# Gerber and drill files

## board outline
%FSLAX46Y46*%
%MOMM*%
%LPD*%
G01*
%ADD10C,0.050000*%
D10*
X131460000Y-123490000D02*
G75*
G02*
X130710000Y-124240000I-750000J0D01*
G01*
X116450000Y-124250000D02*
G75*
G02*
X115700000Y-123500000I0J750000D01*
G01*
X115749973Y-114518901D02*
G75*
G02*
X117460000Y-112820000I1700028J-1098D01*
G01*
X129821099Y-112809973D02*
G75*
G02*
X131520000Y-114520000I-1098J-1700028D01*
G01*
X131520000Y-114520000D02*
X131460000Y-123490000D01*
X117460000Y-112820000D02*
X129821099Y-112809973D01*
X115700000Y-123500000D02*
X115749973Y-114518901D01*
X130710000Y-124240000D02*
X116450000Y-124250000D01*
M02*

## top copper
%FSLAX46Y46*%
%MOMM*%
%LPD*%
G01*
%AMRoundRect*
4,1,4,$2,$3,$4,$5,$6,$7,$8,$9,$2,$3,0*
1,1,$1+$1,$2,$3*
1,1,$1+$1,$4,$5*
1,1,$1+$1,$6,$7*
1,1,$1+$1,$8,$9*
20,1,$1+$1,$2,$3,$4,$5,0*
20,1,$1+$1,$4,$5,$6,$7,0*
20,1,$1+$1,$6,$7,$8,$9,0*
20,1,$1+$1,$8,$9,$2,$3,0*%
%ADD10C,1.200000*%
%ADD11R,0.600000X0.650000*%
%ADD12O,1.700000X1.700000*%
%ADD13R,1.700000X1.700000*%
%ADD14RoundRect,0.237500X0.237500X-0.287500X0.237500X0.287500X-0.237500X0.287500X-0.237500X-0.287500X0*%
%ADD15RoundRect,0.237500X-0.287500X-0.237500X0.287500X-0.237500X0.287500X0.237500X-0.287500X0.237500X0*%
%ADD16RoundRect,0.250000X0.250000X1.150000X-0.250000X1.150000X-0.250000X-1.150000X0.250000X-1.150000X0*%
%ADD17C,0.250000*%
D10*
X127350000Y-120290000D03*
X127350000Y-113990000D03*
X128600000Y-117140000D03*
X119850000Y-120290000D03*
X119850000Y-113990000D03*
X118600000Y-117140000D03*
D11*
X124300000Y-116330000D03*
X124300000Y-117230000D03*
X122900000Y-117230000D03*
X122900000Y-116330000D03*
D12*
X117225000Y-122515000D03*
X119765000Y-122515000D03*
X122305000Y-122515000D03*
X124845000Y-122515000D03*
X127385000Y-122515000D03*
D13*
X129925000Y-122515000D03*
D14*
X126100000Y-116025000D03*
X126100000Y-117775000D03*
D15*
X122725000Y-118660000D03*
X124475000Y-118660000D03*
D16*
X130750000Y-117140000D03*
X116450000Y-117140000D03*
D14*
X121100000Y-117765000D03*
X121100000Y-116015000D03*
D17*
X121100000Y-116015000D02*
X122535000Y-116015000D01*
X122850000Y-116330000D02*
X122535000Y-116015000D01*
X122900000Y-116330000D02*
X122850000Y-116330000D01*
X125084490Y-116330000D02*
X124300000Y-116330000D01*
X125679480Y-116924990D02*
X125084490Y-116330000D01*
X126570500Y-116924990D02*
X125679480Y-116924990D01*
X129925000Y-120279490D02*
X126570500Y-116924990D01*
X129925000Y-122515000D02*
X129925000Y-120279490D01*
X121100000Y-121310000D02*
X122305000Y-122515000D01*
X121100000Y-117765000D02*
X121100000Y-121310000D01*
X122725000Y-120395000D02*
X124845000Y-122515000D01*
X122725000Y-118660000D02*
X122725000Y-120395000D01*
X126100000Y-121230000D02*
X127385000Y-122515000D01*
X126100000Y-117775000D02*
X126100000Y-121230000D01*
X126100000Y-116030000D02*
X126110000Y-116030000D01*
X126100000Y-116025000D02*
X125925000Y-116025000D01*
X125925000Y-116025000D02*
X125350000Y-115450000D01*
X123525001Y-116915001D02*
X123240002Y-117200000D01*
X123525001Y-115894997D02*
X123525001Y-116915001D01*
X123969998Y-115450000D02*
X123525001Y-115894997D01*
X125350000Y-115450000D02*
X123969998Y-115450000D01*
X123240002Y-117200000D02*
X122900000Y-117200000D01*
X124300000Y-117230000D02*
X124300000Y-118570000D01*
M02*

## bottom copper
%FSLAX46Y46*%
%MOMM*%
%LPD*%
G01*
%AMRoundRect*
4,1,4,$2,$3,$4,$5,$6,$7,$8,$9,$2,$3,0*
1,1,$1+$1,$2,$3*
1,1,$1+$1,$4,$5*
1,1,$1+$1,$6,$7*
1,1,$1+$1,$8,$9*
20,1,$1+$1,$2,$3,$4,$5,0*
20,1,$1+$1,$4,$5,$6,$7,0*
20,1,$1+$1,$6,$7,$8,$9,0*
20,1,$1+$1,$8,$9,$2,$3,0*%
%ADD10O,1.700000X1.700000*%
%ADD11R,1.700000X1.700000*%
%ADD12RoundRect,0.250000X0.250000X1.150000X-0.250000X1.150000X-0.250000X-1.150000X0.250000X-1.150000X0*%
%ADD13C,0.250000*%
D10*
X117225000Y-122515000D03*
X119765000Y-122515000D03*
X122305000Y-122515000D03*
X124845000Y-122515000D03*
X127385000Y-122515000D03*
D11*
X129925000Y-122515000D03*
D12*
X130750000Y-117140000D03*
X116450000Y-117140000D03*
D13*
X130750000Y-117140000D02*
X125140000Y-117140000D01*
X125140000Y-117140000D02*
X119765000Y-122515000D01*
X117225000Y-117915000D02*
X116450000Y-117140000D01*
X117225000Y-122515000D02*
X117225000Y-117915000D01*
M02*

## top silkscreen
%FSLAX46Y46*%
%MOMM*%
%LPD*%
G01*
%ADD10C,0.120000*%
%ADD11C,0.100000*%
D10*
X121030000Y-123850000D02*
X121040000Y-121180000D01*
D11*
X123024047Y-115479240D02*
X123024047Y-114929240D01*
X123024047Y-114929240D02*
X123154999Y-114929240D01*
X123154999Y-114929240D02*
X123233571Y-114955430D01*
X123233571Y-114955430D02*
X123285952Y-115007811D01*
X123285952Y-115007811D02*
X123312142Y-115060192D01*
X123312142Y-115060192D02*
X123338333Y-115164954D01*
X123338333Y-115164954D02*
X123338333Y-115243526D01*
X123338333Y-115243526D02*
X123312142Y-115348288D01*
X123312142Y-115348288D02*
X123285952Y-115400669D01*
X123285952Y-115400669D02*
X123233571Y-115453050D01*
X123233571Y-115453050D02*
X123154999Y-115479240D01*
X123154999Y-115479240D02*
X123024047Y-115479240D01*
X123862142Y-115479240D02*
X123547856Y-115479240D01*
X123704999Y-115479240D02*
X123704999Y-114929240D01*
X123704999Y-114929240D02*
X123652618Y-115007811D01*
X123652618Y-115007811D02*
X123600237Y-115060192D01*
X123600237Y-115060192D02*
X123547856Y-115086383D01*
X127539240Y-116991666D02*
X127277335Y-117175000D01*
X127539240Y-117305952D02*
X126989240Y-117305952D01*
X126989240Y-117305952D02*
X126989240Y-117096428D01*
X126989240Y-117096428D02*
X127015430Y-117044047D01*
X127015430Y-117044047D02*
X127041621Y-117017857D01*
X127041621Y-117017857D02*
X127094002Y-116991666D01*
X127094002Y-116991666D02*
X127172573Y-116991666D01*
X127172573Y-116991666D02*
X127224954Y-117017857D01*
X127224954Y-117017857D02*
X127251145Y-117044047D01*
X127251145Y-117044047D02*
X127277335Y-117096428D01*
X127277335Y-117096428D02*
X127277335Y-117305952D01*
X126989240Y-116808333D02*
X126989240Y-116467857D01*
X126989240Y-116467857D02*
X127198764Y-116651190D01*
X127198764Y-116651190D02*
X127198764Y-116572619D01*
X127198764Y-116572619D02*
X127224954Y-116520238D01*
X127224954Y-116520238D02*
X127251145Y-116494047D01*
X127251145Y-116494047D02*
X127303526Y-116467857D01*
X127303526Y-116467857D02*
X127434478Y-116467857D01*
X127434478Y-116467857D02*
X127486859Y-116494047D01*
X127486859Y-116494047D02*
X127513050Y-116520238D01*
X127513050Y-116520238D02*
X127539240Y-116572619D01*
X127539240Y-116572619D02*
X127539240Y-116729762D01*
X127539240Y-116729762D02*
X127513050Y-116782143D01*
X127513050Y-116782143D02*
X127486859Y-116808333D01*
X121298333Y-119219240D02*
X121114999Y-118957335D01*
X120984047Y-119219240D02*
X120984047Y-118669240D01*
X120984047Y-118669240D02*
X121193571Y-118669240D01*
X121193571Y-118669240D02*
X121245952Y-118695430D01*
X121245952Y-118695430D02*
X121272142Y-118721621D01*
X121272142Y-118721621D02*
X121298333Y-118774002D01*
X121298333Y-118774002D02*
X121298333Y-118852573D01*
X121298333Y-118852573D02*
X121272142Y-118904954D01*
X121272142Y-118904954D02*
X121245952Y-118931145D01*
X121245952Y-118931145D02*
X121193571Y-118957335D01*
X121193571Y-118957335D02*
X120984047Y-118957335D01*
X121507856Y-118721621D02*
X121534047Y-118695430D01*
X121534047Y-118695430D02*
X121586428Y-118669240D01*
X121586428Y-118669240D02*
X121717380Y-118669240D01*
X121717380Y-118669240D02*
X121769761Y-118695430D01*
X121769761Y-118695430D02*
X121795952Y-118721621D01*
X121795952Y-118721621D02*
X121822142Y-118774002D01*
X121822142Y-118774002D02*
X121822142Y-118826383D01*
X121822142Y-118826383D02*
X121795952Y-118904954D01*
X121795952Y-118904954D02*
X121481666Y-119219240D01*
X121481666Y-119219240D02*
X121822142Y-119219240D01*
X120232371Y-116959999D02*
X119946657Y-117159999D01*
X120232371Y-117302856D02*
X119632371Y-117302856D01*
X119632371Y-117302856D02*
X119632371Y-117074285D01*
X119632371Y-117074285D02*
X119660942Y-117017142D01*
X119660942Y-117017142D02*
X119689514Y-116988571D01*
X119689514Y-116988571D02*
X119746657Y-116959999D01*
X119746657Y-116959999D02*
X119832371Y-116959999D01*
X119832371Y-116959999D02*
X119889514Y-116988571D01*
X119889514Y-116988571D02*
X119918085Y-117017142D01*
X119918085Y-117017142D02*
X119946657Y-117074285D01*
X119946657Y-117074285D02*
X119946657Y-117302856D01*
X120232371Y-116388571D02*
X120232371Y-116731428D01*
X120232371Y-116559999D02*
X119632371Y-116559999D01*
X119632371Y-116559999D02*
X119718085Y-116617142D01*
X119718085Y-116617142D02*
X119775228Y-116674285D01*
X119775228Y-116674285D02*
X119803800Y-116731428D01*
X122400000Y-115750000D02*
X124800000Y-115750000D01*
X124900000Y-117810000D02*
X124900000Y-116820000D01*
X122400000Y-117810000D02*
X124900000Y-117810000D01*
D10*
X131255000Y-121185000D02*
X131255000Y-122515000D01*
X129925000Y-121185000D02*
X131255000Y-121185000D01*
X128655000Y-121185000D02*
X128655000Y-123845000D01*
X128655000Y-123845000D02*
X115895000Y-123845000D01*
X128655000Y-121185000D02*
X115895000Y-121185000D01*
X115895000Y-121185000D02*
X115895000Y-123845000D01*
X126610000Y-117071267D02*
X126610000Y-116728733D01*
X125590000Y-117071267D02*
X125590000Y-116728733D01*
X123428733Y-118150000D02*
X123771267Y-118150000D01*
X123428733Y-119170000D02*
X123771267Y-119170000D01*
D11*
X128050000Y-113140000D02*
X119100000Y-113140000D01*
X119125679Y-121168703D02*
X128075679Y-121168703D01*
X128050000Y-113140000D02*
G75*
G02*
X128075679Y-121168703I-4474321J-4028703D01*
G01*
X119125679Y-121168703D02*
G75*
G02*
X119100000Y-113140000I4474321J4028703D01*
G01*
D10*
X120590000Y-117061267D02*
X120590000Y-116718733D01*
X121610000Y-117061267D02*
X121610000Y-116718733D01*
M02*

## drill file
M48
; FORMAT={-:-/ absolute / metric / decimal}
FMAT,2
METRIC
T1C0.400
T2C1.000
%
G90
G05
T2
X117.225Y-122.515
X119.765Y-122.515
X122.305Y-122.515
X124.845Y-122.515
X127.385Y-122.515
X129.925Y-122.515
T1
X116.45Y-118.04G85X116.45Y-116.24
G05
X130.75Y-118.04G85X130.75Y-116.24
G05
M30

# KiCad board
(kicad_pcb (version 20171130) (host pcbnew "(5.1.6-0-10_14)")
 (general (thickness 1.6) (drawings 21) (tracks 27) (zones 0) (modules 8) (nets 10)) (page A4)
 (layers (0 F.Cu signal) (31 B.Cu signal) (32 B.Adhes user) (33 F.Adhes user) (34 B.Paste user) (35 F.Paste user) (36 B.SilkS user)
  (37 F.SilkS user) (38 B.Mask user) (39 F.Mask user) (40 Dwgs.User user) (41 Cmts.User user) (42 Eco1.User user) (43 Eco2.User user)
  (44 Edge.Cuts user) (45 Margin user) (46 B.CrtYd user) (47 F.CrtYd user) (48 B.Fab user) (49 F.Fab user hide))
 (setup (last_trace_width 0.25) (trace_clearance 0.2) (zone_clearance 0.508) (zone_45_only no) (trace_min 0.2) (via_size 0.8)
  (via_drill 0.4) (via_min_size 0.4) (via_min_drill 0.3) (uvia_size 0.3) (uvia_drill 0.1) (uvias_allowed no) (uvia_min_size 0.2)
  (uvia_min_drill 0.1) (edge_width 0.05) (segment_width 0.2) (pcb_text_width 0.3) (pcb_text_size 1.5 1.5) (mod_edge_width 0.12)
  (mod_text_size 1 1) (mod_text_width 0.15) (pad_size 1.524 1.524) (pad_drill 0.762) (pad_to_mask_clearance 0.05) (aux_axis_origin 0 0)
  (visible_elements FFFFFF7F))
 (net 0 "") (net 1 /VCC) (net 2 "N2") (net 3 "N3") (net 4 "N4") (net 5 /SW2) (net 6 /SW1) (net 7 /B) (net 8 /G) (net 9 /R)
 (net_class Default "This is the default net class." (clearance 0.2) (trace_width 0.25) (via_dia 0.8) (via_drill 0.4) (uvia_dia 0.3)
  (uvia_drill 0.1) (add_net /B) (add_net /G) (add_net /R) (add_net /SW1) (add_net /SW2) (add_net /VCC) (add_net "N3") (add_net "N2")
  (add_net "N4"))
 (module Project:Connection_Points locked (layer F.Cu) (at 123.6 117.14)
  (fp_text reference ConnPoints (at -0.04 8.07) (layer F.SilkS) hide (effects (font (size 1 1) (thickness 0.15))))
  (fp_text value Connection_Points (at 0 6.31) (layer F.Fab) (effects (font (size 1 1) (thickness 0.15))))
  (pad "" smd circle (at 3.75 3.15) (size 1.2 1.2) (layers F.Cu F.Paste F.Mask))
  (pad "" smd circle (at 3.75 -3.15) (size 1.2 1.2) (layers F.Cu F.Paste F.Mask))
  (pad "" smd circle (at 5 0) (size 1.2 1.2) (layers F.Cu F.Paste F.Mask))
  (pad "" smd circle (at -3.75 3.15) (size 1.2 1.2) (layers F.Cu F.Paste F.Mask))
  (pad "" smd circle (at -3.75 -3.15) (size 1.2 1.2) (layers F.Cu F.Paste F.Mask))
  (pad "" smd circle (at -5 0) (size 1.2 1.2) (layers F.Cu F.Paste F.Mask)))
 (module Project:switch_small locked (layer B.Cu) (at 118.42 120.41 180)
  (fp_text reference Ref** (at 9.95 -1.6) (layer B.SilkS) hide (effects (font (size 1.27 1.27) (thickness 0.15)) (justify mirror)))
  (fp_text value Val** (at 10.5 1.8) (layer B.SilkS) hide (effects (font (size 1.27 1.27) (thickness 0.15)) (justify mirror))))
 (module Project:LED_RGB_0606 (layer F.Cu) (at 123.6 116.78)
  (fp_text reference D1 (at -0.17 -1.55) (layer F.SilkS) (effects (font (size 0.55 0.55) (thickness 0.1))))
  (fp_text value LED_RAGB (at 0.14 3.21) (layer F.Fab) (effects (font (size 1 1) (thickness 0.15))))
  (fp_line (start -1.2 -1.03) (end 1.2 -1.03) (layer F.SilkS) (width 0.1))
  (fp_line (start 1.3 1.03) (end 1.3 0.04) (layer F.SilkS) (width 0.1))
  (fp_line (start -1.2 1.03) (end 1.3 1.03) (layer F.SilkS) (width 0.1))
  (pad 4 smd rect (at 0.7 -0.45) (size 0.6 0.65) (layers F.Cu F.Paste F.Mask) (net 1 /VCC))
  (pad 2 smd rect (at 0.7 0.45) (size 0.6 0.65) (layers F.Cu F.Paste F.Mask) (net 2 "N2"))
  (pad 1 smd rect (at -0.7 0.45) (size 0.6 0.65) (layers F.Cu F.Paste F.Mask) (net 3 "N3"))
  (pad 3 smd rect (at -0.7 -0.45) (size 0.6 0.65) (layers F.Cu F.Paste F.Mask) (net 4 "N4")))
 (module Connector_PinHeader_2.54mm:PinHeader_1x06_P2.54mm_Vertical (layer F.Cu) (at 129.925 122.515 270)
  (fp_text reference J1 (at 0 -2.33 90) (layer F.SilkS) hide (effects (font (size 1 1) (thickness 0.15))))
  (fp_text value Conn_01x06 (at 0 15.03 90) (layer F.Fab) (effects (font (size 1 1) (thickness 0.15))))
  (fp_line (start -1.33 -1.33) (end 0 -1.33) (layer F.SilkS) (width 0.12))
  (fp_line (start -1.33 0) (end -1.33 -1.33) (layer F.SilkS) (width 0.12))
  (fp_line (start -1.33 1.27) (end 1.33 1.27) (layer F.SilkS) (width 0.12))
  (fp_line (start 1.33 1.27) (end 1.33 14.03) (layer F.SilkS) (width 0.12))
  (fp_line (start -1.33 1.27) (end -1.33 14.03) (layer F.SilkS) (width 0.12))
  (fp_line (start -1.33 14.03) (end 1.33 14.03) (layer F.SilkS) (width 0.12))
  (pad 6 thru_hole oval (at 0 12.7 270) (size 1.7 1.7) (drill 1) (layers *.Cu *.Mask) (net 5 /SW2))
  (pad 5 thru_hole oval (at 0 10.16 270) (size 1.7 1.7) (drill 1) (layers *.Cu *.Mask) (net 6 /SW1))
  (pad 4 thru_hole oval (at 0 7.62 270) (size 1.7 1.7) (drill 1) (layers *.Cu *.Mask) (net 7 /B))
  (pad 3 thru_hole oval (at 0 5.08 270) (size 1.7 1.7) (drill 1) (layers *.Cu *.Mask) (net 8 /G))
  (pad 2 thru_hole oval (at 0 2.54 270) (size 1.7 1.7) (drill 1) (layers *.Cu *.Mask) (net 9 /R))
  (pad 1 thru_hole rect (at 0 0 270) (size 1.7 1.7) (drill 1) (layers *.Cu *.Mask) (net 1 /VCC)))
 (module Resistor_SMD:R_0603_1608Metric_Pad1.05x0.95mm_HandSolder (layer F.Cu) (at 126.1 116.9 90)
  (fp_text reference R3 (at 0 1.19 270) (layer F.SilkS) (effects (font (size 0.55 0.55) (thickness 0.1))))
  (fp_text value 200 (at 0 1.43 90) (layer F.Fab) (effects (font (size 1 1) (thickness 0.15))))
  (fp_line (start -0.171267 0.51) (end 0.171267 0.51) (layer F.SilkS) (width 0.12))
  (fp_line (start -0.171267 -0.51) (end 0.171267 -0.51) (layer F.SilkS) (width 0.12))
  (pad 2 smd roundrect (at 0.875 0 90) (size 1.05 0.95) (layers F.Cu F.Paste F.Mask) (roundrect_rratio 0.25) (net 3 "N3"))
  (pad 1 smd roundrect (at -0.875 0 90) (size 1.05 0.95) (layers F.Cu F.Paste F.Mask) (roundrect_rratio 0.25) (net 9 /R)))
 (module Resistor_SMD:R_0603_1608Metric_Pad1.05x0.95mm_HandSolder (layer F.Cu) (at 123.6 118.66)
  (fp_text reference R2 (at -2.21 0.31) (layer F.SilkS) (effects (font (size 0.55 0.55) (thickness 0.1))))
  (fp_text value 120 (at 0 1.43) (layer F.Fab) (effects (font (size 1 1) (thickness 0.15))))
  (fp_line (start -0.171267 -0.51) (end 0.171267 -0.51) (layer F.SilkS) (width 0.12))
  (fp_line (start -0.171267 0.51) (end 0.171267 0.51) (layer F.SilkS) (width 0.12))
  (pad 1 smd roundrect (at -0.875 0) (size 1.05 0.95) (layers F.Cu F.Paste F.Mask) (roundrect_rratio 0.25) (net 8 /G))
  (pad 2 smd roundrect (at 0.875 0) (size 1.05 0.95) (layers F.Cu F.Paste F.Mask) (roundrect_rratio 0.25) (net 2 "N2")))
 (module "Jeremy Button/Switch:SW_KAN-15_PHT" (layer F.Cu) (at 123.6 117.14 180)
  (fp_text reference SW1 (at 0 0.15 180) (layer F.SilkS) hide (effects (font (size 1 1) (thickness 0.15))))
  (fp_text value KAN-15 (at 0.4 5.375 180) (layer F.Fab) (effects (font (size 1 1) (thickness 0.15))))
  (fp_line (start -4.45 4) (end 4.5 4) (layer F.SilkS) (width 0.1))
  (fp_line (start 4.474321 -4.028703) (end -4.475679 -4.028703) (layer F.SilkS) (width 0.1))
  (fp_arc (start 0.024321 -0.028703) (end -4.475679 -4.028703) (angle -83.63358372) (layer F.SilkS) (width 0.1))
  (fp_arc (start 0 0) (end 4.5 4) (angle -83.63358372) (layer F.SilkS) (width 0.1))
  (pad 1 thru_hole roundrect (at -7.15 0 180) (size 1 2.8) (drill oval 0.4 2.2) (layers *.Cu *.Mask) (roundrect_rratio 0.25) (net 6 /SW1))
  (pad 2 thru_hole roundrect (at 7.15 0 180) (size 1 2.8) (drill oval 0.4 2.2) (layers *.Cu *.Mask) (roundrect_rratio 0.25) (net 5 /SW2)))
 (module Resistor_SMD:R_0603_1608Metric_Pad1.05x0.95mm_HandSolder (layer F.Cu) (at 121.1 116.89 90)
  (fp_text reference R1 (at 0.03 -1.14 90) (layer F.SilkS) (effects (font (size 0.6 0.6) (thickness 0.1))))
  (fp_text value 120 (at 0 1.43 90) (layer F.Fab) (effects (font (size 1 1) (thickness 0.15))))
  (fp_line (start -0.171267 -0.51) (end 0.171267 -0.51) (layer F.SilkS) (width 0.12))
  (fp_line (start -0.171267 0.51) (end 0.171267 0.51) (layer F.SilkS) (width 0.12))
  (pad 1 smd roundrect (at -0.875 0 90) (size 1.05 0.95) (layers F.Cu F.Paste F.Mask) (roundrect_rratio 0.25) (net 7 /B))
  (pad 2 smd roundrect (at 0.875 0 90) (size 1.05 0.95) (layers F.Cu F.Paste F.Mask) (roundrect_rratio 0.25) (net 4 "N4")))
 (gr_arc (start 130.71 123.49) (end 130.71 124.24) (angle -90) (layer Edge.Cuts) (width 0.05))
 (gr_arc (start 116.45 123.5) (end 115.7 123.5) (angle -90) (layer Edge.Cuts) (width 0.05))
 (gr_arc (start 117.450001 114.519999) (end 117.46 112.82) (angle -90.3) (layer Edge.Cuts) (width 0.05))
 (gr_arc (start 129.820001 114.510001) (end 131.52 114.52) (angle -90.3) (layer Edge.Cuts) (width 0.05))
 (gr_line (start 121.03 123.85) (end 121.04 121.18) (layer F.SilkS) (width 0.12))
 (gr_line (start 131.52 114.52) (end 131.46 123.49) (layer Edge.Cuts) (width 0.05))
 (gr_line (start 117.46 112.82) (end 129.821099 112.809973) (layer Edge.Cuts) (width 0.05))
 (gr_line (start 115.7 123.5) (end 115.749973 114.518901) (layer Edge.Cuts) (width 0.05))
 (gr_line (start 130.71 124.24) (end 116.45 124.25) (layer Edge.Cuts) (width 0.05))
 (segment (start 121.1 116.015) (end 122.535 116.015) (width 0.25) (layer F.Cu) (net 4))
 (segment (start 122.85 116.33) (end 122.535 116.015) (width 0.25) (layer F.Cu) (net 4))
 (segment (start 122.9 116.33) (end 122.85 116.33) (width 0.25) (layer F.Cu) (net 4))
 (segment (start 125.08449 116.33) (end 124.3 116.33) (width 0.25) (layer F.Cu) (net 1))
 (segment (start 125.67948 116.92499) (end 125.08449 116.33) (width 0.25) (layer F.Cu) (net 1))
 (segment (start 126.5705 116.92499) (end 125.67948 116.92499) (width 0.25) (layer F.Cu) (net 1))
 (segment (start 129.925 120.27949) (end 126.5705 116.92499) (width 0.25) (layer F.Cu) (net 1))
 (segment (start 129.925 122.515) (end 129.925 120.27949) (width 0.25) (layer F.Cu) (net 1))
 (segment (start 121.1 121.31) (end 122.305 122.515) (width 0.25) (layer F.Cu) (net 7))
 (segment (start 121.1 117.765) (end 121.1 121.31) (width 0.25) (layer F.Cu) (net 7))
 (segment (start 122.725 120.395) (end 124.845 122.515) (width 0.25) (layer F.Cu) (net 8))
 (segment (start 122.725 118.66) (end 122.725 120.395) (width 0.25) (layer F.Cu) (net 8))
 (segment (start 126.1 121.23) (end 127.385 122.515) (width 0.25) (layer F.Cu) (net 9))
 (segment (start 126.1 117.775) (end 126.1 121.23) (width 0.25) (layer F.Cu) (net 9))
 (segment (start 130.75 117.14) (end 125.14 117.14) (width 0.25) (layer B.Cu) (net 6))
 (segment (start 125.14 117.14) (end 119.765 122.515) (width 0.25) (layer B.Cu) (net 6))
 (segment (start 117.225 117.915) (end 116.45 117.14) (width 0.25) (layer B.Cu) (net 5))
 (segment (start 117.225 122.515) (end 117.225 117.915) (width 0.25) (layer B.Cu) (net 5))
 (segment (start 126.1 116.03) (end 126.11 116.03) (width 0.25) (layer F.Cu) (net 3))
 (segment (start 126.1 116.025) (end 125.925 116.025) (width 0.25) (layer F.Cu) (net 3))
 (segment (start 125.925 116.025) (end 125.35 115.45) (width 0.25) (layer F.Cu) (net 3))
 (segment (start 123.525001 116.915001) (end 123.240002 117.2) (width 0.25) (layer F.Cu) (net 3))
 (segment (start 123.525001 115.894997) (end 123.525001 116.915001) (width 0.25) (layer F.Cu) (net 3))
 (segment (start 123.969998 115.45) (end 123.525001 115.894997) (width 0.25) (layer F.Cu) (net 3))
 (segment (start 125.35 115.45) (end 123.969998 115.45) (width 0.25) (layer F.Cu) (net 3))
 (segment (start 123.240002 117.2) (end 122.9 117.2) (width 0.25) (layer F.Cu) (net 3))
 (segment (start 124.3 117.23) (end 124.3 118.57) (width 0.25) (layer F.Cu) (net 2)))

